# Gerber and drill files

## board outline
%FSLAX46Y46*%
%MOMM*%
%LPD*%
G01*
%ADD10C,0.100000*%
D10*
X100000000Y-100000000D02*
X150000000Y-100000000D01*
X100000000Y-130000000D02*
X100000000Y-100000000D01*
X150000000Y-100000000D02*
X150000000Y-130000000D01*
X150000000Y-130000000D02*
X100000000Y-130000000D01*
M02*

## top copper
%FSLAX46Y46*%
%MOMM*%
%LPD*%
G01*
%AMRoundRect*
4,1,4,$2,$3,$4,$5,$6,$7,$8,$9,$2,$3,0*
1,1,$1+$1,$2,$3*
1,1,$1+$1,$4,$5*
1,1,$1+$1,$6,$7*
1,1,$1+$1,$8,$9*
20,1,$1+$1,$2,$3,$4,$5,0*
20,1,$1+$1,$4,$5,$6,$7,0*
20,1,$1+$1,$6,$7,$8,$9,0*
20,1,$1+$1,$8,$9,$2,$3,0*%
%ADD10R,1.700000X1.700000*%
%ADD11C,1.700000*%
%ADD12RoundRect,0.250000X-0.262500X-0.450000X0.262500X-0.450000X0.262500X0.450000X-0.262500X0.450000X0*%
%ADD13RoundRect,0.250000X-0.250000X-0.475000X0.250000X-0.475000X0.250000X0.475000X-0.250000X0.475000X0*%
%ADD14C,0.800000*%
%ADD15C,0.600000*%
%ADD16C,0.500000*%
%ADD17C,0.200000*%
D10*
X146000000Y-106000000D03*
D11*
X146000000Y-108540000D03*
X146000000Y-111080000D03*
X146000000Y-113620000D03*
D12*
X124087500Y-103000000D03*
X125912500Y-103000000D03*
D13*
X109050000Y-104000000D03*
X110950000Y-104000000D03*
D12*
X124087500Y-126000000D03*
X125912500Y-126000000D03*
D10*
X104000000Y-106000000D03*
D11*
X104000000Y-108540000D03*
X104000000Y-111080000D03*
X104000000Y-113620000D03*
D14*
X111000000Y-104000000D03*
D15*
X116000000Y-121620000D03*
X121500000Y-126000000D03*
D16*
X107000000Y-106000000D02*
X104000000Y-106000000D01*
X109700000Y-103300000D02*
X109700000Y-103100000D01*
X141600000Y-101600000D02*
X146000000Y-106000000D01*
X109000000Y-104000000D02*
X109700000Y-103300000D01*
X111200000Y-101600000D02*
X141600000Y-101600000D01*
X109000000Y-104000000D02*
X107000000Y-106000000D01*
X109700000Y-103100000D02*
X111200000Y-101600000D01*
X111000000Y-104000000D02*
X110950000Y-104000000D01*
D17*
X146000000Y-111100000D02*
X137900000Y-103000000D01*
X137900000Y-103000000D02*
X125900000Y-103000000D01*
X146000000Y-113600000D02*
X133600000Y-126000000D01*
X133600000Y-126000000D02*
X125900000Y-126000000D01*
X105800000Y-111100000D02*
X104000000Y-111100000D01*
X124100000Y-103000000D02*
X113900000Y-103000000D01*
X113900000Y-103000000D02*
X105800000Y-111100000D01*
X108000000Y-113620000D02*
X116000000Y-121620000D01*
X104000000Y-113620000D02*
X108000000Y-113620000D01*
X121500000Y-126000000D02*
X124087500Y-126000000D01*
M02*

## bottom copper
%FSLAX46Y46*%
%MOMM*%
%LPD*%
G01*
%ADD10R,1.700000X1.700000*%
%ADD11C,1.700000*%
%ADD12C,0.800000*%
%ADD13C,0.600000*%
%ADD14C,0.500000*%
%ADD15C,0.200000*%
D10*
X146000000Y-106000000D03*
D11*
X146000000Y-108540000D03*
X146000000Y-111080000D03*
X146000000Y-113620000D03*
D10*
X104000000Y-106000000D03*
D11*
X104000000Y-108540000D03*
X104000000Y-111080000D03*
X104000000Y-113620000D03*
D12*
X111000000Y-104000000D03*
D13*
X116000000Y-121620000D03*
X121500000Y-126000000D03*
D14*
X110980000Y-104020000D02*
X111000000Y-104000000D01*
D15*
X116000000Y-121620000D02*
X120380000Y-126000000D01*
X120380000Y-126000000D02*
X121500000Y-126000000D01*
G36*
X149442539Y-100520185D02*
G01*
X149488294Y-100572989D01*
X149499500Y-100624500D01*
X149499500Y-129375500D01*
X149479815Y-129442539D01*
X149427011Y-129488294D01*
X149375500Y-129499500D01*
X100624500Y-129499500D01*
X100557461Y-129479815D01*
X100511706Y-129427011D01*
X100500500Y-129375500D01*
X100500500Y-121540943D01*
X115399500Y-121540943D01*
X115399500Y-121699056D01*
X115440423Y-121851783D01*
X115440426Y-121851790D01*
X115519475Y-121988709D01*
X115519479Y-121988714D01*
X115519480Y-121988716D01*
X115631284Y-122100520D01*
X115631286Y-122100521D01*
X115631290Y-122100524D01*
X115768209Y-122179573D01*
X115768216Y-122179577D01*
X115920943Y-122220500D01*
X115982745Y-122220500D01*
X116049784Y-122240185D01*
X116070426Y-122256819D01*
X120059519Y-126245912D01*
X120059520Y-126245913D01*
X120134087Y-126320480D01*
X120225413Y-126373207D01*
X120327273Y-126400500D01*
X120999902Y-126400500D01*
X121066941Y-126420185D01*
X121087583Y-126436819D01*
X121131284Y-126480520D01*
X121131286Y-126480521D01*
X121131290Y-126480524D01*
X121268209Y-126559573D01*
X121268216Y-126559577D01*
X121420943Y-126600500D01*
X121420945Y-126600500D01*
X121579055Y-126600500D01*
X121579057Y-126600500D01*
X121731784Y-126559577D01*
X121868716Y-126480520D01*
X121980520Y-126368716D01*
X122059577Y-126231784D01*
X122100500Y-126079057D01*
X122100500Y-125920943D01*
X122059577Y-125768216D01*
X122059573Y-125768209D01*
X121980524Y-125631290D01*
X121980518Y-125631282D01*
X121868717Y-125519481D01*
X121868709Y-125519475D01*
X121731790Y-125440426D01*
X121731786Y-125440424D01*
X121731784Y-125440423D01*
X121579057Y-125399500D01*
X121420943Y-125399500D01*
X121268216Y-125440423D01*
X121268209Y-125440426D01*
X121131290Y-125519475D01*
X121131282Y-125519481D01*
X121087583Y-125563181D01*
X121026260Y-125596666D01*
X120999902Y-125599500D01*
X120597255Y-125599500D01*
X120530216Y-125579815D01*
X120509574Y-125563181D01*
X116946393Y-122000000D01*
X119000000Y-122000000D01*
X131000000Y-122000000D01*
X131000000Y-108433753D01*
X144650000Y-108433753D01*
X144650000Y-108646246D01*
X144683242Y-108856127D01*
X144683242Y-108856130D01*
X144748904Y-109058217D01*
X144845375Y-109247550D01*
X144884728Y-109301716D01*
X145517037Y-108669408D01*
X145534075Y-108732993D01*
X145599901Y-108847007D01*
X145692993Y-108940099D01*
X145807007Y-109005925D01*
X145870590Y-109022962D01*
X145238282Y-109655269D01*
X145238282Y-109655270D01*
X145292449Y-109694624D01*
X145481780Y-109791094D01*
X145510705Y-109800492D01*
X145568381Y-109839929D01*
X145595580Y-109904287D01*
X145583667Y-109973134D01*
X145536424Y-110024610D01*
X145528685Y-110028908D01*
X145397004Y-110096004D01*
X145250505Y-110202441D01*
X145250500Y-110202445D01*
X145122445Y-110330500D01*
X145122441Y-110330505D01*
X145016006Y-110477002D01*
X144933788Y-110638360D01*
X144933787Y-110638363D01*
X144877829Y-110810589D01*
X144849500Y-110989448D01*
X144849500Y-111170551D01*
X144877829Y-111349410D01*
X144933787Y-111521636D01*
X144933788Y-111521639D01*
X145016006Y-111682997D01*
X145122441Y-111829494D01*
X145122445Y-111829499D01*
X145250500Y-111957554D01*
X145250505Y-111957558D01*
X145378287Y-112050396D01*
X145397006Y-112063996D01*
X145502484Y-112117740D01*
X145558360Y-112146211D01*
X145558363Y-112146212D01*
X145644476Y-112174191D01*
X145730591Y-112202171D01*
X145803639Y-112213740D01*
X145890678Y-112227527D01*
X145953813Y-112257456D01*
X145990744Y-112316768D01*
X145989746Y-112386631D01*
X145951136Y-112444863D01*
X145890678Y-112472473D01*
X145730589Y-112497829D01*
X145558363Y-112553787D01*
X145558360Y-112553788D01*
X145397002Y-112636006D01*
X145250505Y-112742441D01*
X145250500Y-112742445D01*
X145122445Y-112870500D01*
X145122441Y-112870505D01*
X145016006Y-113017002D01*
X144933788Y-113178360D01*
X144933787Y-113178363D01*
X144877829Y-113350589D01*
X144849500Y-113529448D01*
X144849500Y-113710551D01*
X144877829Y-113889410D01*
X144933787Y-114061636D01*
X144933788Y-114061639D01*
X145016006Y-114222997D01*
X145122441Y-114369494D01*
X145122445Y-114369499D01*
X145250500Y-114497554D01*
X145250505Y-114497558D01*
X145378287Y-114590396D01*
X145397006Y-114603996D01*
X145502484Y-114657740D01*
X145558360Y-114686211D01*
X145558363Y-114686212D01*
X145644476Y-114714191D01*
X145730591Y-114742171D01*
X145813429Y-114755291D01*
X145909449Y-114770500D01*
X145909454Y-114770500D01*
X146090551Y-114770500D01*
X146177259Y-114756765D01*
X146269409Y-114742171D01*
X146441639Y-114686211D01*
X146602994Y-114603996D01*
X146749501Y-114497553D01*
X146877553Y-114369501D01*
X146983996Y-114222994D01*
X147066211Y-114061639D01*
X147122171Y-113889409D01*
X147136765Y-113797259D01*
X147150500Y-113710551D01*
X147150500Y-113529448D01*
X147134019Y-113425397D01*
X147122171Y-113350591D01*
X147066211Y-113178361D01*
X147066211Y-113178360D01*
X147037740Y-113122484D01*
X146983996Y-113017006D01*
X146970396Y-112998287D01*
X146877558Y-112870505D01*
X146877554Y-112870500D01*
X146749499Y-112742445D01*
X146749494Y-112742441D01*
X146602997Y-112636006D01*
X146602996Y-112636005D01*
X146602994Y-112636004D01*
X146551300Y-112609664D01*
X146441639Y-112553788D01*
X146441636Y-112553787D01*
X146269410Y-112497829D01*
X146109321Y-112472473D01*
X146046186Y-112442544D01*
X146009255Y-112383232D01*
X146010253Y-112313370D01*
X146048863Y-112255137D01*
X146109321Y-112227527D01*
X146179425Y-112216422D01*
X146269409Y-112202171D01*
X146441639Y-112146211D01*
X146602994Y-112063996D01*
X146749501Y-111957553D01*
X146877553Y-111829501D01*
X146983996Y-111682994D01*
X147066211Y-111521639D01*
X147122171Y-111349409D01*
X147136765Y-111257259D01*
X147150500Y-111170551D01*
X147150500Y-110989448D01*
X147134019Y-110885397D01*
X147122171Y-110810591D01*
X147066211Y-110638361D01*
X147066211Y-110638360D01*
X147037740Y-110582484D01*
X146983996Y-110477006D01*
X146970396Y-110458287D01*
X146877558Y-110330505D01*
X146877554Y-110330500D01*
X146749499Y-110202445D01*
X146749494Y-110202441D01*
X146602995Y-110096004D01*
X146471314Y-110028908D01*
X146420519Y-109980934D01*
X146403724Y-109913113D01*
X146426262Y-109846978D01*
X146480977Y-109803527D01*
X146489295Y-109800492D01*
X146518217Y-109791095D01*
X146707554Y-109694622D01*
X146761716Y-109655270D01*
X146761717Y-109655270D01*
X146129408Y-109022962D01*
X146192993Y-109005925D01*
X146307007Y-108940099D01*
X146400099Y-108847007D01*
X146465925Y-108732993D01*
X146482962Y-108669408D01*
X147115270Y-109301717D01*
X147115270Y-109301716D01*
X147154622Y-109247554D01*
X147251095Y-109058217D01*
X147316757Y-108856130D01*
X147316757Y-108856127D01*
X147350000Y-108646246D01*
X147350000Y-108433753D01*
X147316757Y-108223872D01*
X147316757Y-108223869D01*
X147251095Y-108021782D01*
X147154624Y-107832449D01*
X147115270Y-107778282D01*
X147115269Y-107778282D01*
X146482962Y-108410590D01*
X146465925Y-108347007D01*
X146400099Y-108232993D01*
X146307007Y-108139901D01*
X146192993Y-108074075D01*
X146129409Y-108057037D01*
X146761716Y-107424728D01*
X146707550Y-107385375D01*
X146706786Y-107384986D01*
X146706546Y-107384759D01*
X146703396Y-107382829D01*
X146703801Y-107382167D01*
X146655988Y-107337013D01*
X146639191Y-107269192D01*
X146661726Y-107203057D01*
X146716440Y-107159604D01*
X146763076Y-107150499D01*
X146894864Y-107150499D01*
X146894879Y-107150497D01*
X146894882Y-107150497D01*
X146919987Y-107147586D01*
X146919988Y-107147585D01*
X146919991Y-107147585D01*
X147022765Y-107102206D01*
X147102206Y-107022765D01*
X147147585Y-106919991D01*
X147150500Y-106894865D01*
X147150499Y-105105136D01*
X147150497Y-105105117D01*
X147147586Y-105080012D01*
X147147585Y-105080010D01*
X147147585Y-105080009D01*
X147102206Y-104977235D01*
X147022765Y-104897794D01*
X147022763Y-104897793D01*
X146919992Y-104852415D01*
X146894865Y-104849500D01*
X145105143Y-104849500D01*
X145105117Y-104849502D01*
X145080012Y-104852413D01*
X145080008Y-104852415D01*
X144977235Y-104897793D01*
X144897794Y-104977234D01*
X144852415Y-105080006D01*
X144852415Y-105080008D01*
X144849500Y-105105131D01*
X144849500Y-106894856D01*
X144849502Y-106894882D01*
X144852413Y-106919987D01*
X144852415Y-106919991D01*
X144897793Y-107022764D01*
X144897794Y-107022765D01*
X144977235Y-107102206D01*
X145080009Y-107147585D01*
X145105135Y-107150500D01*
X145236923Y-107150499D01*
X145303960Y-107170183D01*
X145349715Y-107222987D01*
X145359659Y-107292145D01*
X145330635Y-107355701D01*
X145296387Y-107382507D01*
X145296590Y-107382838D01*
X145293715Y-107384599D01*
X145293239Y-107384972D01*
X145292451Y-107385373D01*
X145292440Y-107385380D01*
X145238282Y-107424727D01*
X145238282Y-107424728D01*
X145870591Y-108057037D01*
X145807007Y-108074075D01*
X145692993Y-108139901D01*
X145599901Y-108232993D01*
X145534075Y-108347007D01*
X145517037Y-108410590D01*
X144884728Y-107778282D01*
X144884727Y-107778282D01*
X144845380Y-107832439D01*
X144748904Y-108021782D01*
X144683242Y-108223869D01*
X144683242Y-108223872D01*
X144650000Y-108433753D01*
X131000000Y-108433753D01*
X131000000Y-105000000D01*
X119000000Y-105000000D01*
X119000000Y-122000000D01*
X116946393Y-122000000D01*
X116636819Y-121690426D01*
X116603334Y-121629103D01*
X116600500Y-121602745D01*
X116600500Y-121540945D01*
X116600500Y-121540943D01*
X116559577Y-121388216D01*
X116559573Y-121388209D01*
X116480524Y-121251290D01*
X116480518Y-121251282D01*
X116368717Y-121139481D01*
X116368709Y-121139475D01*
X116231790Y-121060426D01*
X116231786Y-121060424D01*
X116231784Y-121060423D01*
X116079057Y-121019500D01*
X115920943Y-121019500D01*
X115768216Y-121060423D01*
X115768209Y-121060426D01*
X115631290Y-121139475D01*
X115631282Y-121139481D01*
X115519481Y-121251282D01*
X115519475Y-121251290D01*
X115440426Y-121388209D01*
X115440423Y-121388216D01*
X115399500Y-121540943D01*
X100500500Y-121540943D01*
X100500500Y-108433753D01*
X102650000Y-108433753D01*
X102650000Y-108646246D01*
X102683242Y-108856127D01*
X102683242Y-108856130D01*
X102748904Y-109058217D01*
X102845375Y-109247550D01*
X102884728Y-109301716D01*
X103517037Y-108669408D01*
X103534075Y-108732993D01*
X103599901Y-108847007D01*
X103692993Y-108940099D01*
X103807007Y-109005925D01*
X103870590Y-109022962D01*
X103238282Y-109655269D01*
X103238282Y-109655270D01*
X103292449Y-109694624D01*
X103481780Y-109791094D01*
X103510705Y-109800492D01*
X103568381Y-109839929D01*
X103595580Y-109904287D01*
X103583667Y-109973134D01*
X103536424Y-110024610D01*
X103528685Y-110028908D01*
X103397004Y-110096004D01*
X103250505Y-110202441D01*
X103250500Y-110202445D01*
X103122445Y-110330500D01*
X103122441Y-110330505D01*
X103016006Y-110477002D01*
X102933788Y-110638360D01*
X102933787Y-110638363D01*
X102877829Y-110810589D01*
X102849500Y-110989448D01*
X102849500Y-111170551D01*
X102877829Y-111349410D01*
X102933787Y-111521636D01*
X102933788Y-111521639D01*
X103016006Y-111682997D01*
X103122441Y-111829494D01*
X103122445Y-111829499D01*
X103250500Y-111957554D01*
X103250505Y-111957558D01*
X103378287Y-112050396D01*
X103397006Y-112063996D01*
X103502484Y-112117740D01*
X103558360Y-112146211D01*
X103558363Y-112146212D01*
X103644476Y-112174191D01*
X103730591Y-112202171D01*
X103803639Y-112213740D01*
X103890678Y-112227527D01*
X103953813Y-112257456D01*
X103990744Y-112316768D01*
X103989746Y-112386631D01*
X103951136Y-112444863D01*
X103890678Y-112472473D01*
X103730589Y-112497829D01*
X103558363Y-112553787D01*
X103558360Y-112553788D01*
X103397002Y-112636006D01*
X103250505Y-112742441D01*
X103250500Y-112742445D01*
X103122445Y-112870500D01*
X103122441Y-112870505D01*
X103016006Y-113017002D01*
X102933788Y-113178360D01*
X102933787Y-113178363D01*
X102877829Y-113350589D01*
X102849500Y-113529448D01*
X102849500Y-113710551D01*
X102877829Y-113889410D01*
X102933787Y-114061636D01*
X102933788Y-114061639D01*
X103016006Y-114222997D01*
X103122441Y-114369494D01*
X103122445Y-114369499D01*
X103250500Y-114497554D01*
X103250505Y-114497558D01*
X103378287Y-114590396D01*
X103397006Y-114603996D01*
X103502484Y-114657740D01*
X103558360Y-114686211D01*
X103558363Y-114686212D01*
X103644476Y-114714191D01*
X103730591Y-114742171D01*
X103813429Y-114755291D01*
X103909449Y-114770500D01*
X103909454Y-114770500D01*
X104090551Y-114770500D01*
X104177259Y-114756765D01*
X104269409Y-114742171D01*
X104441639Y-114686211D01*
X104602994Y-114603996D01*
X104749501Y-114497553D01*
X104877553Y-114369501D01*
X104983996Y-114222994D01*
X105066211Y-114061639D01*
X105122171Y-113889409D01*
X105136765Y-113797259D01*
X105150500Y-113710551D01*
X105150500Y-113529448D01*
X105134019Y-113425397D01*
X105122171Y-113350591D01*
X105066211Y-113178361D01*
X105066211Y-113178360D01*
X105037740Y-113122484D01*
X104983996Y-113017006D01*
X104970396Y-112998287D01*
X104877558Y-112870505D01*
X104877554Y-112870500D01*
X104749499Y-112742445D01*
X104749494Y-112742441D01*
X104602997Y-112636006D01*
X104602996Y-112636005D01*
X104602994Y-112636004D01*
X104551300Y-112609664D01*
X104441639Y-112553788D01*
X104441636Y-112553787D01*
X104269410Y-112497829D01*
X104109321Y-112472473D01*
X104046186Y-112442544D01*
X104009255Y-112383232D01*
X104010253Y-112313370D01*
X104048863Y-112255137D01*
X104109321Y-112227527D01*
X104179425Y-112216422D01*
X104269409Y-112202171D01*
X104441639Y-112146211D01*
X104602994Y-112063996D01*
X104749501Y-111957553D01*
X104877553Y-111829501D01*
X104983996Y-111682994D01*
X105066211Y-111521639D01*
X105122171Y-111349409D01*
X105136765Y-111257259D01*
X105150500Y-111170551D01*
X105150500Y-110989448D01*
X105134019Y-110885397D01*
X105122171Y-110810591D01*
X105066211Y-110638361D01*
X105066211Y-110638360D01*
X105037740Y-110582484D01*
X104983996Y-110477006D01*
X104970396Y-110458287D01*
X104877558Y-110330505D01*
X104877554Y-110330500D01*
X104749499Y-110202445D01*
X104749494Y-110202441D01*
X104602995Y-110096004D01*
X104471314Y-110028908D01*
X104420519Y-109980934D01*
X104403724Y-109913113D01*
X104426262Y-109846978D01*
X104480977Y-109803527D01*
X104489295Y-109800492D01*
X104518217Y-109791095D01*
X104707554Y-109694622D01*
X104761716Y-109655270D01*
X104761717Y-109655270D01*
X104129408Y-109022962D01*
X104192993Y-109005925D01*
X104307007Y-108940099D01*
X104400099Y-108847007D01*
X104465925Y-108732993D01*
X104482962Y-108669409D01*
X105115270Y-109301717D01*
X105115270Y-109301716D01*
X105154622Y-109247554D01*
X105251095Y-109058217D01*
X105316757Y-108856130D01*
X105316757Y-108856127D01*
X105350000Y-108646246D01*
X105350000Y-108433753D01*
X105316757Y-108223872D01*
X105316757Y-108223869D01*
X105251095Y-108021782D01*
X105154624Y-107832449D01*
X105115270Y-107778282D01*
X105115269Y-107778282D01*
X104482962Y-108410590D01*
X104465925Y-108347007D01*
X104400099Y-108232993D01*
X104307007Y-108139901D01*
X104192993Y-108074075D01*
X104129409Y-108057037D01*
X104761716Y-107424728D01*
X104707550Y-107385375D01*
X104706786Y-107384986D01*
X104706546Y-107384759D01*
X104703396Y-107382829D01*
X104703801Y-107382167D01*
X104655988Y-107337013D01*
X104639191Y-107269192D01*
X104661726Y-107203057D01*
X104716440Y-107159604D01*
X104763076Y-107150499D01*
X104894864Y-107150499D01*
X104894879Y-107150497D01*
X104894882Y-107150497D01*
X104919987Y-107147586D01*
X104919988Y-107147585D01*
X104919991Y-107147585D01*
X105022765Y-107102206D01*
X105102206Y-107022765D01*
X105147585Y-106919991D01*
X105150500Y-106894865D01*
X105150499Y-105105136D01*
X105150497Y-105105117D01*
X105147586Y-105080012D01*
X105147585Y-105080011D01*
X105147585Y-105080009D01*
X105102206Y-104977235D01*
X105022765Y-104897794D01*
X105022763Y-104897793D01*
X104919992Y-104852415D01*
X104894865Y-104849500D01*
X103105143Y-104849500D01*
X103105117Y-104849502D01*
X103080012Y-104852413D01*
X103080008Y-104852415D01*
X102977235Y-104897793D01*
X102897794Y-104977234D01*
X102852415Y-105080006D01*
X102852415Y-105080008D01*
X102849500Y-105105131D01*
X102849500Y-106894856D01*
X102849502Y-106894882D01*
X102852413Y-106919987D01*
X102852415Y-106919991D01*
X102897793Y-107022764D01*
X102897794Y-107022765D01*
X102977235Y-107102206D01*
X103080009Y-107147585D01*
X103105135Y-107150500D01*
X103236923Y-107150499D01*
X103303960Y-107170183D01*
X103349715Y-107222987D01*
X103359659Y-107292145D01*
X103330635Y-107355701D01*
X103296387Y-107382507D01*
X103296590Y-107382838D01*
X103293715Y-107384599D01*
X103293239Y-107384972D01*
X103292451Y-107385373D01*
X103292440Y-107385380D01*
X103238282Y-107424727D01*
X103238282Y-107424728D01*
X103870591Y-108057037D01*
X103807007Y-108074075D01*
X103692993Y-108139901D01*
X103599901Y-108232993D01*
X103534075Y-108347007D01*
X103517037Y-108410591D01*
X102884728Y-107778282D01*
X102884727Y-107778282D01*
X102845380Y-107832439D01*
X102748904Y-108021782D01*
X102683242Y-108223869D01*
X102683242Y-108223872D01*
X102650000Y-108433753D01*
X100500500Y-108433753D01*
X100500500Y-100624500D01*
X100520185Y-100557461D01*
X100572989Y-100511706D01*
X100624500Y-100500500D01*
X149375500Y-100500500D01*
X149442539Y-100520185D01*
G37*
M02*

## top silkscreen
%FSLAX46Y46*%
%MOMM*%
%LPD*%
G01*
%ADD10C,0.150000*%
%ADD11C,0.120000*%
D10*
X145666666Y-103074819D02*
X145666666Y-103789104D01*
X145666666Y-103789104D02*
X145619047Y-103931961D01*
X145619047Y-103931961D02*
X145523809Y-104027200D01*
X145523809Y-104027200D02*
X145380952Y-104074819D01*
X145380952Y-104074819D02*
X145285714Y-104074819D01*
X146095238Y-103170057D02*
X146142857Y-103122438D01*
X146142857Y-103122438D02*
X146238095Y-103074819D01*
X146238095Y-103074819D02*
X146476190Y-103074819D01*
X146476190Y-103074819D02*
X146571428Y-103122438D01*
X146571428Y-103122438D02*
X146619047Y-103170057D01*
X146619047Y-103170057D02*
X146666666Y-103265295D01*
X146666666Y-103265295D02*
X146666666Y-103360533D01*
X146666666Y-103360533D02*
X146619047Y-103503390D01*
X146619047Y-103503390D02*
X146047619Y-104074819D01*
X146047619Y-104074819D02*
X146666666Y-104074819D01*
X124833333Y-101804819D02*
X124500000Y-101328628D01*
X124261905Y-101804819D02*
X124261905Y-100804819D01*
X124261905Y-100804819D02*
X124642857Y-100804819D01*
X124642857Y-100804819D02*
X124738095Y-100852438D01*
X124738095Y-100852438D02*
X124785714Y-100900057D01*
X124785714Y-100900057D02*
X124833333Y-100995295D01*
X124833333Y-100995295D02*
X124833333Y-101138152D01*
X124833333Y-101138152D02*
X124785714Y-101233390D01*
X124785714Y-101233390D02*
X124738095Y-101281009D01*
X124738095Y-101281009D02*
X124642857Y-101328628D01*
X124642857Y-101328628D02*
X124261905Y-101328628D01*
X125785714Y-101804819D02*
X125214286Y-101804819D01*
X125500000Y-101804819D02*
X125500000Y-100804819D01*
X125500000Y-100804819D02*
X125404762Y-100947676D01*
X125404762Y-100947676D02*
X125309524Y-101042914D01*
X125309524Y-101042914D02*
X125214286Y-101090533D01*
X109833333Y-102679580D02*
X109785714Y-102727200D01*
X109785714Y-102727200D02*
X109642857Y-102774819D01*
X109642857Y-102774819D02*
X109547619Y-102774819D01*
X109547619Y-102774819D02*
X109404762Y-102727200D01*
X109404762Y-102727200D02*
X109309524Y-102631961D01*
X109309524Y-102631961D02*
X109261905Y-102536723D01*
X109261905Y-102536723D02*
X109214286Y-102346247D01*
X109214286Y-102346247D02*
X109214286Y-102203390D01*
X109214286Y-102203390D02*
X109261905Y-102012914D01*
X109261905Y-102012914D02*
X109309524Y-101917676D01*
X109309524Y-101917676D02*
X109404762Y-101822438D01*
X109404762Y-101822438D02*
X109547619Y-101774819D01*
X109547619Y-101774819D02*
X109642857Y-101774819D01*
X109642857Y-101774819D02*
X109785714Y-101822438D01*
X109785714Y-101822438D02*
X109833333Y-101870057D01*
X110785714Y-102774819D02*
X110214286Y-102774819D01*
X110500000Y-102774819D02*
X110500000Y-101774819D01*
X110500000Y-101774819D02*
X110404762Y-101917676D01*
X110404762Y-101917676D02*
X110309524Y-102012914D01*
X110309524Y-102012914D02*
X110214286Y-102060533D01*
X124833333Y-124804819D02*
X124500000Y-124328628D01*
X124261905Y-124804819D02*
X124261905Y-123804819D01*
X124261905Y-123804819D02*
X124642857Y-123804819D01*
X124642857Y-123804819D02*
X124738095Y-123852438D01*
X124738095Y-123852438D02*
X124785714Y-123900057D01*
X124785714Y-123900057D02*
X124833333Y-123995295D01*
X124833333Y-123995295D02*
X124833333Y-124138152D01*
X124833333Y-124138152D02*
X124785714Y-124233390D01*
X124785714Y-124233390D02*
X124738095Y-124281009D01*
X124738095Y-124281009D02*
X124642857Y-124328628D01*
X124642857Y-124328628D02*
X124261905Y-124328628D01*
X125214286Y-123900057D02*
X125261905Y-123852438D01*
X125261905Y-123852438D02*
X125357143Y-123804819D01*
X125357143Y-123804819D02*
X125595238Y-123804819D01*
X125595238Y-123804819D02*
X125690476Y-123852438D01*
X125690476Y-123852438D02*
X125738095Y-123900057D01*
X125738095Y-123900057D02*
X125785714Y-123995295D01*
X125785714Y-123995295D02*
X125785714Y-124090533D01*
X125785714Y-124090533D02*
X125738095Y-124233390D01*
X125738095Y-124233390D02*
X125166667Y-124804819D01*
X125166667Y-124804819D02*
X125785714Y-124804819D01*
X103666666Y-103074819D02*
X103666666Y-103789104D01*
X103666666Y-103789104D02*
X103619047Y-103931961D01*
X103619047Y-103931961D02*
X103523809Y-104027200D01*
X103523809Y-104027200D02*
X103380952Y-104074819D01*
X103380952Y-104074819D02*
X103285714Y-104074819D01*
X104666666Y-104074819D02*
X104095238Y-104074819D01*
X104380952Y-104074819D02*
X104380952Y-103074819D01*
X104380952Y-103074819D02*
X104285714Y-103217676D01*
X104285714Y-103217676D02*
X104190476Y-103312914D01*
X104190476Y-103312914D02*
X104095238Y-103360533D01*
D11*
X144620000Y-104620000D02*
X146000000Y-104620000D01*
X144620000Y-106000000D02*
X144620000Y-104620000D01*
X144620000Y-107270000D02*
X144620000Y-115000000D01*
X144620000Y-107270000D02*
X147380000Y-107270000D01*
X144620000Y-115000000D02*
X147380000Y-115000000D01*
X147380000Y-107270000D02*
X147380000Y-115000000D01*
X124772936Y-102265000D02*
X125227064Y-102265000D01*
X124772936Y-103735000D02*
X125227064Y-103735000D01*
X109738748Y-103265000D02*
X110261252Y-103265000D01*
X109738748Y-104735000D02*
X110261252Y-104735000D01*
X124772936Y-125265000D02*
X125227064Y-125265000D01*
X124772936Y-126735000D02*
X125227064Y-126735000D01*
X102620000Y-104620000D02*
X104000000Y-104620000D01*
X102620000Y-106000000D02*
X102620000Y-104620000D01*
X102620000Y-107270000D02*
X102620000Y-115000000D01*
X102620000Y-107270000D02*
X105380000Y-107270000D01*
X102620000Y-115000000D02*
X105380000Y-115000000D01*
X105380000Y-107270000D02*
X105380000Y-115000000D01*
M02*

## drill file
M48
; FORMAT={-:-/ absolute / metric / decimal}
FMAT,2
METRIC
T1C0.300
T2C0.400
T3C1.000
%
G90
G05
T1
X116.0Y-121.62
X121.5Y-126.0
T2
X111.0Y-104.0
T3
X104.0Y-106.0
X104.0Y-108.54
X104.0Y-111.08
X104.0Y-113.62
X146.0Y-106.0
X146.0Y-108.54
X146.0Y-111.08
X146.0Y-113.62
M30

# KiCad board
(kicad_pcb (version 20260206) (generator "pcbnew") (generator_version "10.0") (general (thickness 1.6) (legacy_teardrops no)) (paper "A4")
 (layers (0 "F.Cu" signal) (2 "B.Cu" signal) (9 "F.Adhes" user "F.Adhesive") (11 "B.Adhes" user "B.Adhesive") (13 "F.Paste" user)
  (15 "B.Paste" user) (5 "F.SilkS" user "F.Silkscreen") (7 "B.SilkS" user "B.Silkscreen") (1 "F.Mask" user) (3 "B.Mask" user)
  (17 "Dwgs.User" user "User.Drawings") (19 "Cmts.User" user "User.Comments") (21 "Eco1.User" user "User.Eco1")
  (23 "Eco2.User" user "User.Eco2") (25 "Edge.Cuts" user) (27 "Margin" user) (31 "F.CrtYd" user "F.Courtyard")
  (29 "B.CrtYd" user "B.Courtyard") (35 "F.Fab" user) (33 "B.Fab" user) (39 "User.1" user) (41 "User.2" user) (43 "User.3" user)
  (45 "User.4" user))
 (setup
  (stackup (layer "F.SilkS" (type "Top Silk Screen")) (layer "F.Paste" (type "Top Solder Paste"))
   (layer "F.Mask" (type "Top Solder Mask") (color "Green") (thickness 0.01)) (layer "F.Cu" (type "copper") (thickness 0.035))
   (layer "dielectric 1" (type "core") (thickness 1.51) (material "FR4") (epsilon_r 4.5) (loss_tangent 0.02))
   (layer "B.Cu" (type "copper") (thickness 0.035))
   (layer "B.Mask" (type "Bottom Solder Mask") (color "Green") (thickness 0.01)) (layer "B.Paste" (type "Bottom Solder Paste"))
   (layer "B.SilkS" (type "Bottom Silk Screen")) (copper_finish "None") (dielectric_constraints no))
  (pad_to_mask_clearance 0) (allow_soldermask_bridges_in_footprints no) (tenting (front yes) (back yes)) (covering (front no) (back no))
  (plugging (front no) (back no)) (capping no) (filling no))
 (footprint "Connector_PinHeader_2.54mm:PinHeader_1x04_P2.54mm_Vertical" (layer "F.Cu") (at 146 106)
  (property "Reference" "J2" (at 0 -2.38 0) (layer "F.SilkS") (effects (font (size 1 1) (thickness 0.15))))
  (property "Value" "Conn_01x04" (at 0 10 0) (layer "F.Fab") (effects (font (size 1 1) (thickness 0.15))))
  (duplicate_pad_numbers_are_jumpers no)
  (fp_line (start -1.38 -1.38) (end 0 -1.38) (stroke (width 0.12) (type solid)) (layer "F.SilkS"))
  (fp_line (start -1.38 0) (end -1.38 -1.38) (stroke (width 0.12) (type solid)) (layer "F.SilkS"))
  (fp_line (start -1.38 1.27) (end -1.38 9) (stroke (width 0.12) (type solid)) (layer "F.SilkS"))
  (fp_line (start -1.38 1.27) (end 1.38 1.27) (stroke (width 0.12) (type solid)) (layer "F.SilkS"))
  (fp_line (start -1.38 9) (end 1.38 9) (stroke (width 0.12) (type solid)) (layer "F.SilkS"))
  (fp_line (start 1.38 1.27) (end 1.38 9) (stroke (width 0.12) (type solid)) (layer "F.SilkS"))
  (pad "1" thru_hole rect (at 0 0) (size 1.7 1.7) (drill 1) (layers "*.Cu" "*.Mask") (remove_unused_layers no) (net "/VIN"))
  (pad "2" thru_hole circle (at 0 2.54) (size 1.7 1.7) (drill 1) (layers "*.Cu" "*.Mask") (remove_unused_layers no) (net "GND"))
  (pad "3" thru_hole circle (at 0 5.08) (size 1.7 1.7) (drill 1) (layers "*.Cu" "*.Mask") (remove_unused_layers no) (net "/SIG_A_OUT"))
  (pad "4" thru_hole circle (at 0 7.62) (size 1.7 1.7) (drill 1) (layers "*.Cu" "*.Mask") (remove_unused_layers no) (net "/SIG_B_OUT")))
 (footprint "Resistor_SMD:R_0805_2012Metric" (layer "F.Cu") (at 125 103)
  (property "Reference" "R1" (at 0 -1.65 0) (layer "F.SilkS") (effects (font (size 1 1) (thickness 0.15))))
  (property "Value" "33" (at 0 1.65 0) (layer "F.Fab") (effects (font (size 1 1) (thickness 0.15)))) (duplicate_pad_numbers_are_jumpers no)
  (fp_line (start -0.227064 -0.735) (end 0.227064 -0.735) (stroke (width 0.12) (type solid)) (layer "F.SilkS"))
  (fp_line (start -0.227064 0.735) (end 0.227064 0.735) (stroke (width 0.12) (type solid)) (layer "F.SilkS"))
  (pad "1" smd roundrect (at -0.9125 0) (size 1.025 1.4) (layers "F.Cu" "F.Mask" "F.Paste") (roundrect_rratio 0.243902) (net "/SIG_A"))
  (pad "2" smd roundrect (at 0.9125 0) (size 1.025 1.4) (layers "F.Cu" "F.Mask" "F.Paste") (roundrect_rratio 0.243902) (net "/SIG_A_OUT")))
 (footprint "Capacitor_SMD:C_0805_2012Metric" (layer "F.Cu") (at 110 104)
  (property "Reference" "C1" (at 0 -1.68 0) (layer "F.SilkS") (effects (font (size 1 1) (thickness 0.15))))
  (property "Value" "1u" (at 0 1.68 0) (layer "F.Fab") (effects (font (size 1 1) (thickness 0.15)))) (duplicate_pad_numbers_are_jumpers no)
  (fp_line (start -0.261252 -0.735) (end 0.261252 -0.735) (stroke (width 0.12) (type solid)) (layer "F.SilkS"))
  (fp_line (start -0.261252 0.735) (end 0.261252 0.735) (stroke (width 0.12) (type solid)) (layer "F.SilkS"))
  (pad "1" smd roundrect (at -0.95 0) (size 1 1.45) (layers "F.Cu" "F.Mask" "F.Paste") (roundrect_rratio 0.25) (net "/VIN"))
  (pad "2" smd roundrect (at 0.95 0) (size 1 1.45) (layers "F.Cu" "F.Mask" "F.Paste") (roundrect_rratio 0.25) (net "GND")))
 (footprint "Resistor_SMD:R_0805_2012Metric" (layer "F.Cu") (at 125 126)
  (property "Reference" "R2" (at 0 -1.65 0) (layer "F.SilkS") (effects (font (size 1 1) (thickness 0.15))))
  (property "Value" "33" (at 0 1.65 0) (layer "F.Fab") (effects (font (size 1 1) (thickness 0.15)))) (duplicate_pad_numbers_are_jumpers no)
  (fp_line (start -0.227064 -0.735) (end 0.227064 -0.735) (stroke (width 0.12) (type solid)) (layer "F.SilkS"))
  (fp_line (start -0.227064 0.735) (end 0.227064 0.735) (stroke (width 0.12) (type solid)) (layer "F.SilkS"))
  (pad "1" smd roundrect (at -0.9125 0) (size 1.025 1.4) (layers "F.Cu" "F.Mask" "F.Paste") (roundrect_rratio 0.243902) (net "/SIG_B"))
  (pad "2" smd roundrect (at 0.9125 0) (size 1.025 1.4) (layers "F.Cu" "F.Mask" "F.Paste") (roundrect_rratio 0.243902) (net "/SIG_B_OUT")))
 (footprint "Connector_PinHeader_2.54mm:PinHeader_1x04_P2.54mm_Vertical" (layer "F.Cu") (at 104 106)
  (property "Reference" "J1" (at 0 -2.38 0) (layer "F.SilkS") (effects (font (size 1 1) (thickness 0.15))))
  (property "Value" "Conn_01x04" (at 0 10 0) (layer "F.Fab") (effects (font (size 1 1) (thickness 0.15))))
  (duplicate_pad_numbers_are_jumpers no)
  (fp_line (start -1.38 -1.38) (end 0 -1.38) (stroke (width 0.12) (type solid)) (layer "F.SilkS"))
  (fp_line (start -1.38 0) (end -1.38 -1.38) (stroke (width 0.12) (type solid)) (layer "F.SilkS"))
  (fp_line (start -1.38 1.27) (end -1.38 9) (stroke (width 0.12) (type solid)) (layer "F.SilkS"))
  (fp_line (start -1.38 1.27) (end 1.38 1.27) (stroke (width 0.12) (type solid)) (layer "F.SilkS"))
  (fp_line (start -1.38 9) (end 1.38 9) (stroke (width 0.12) (type solid)) (layer "F.SilkS"))
  (fp_line (start 1.38 1.27) (end 1.38 9) (stroke (width 0.12) (type solid)) (layer "F.SilkS"))
  (pad "1" thru_hole rect (at 0 0) (size 1.7 1.7) (drill 1) (layers "*.Cu" "*.Mask") (remove_unused_layers no) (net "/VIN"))
  (pad "2" thru_hole circle (at 0 2.54) (size 1.7 1.7) (drill 1) (layers "*.Cu" "*.Mask") (remove_unused_layers no) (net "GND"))
  (pad "3" thru_hole circle (at 0 5.08) (size 1.7 1.7) (drill 1) (layers "*.Cu" "*.Mask") (remove_unused_layers no) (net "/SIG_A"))
  (pad "4" thru_hole circle (at 0 7.62) (size 1.7 1.7) (drill 1) (layers "*.Cu" "*.Mask") (remove_unused_layers no) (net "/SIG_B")))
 (gr_line (start 100 100) (end 150 100) (stroke (width 0.1) (type default)) (layer "Edge.Cuts"))
 (gr_line (start 100 130) (end 100 100) (stroke (width 0.1) (type default)) (layer "Edge.Cuts"))
 (gr_line (start 150 100) (end 150 130) (stroke (width 0.1) (type default)) (layer "Edge.Cuts"))
 (gr_line (start 150 130) (end 100 130) (stroke (width 0.1) (type default)) (layer "Edge.Cuts"))
 (segment (start 107 106) (end 104 106) (width 0.5) (layer "F.Cu") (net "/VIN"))
 (segment (start 109.7 103.3) (end 109.7 103.1) (width 0.5) (layer "F.Cu") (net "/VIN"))
 (segment (start 141.6 101.6) (end 146 106) (width 0.5) (layer "F.Cu") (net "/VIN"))
 (segment (start 109 104) (end 109.7 103.3) (width 0.5) (layer "F.Cu") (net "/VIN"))
 (segment (start 111.2 101.6) (end 141.6 101.6) (width 0.5) (layer "F.Cu") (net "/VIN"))
 (segment (start 109 104) (end 107 106) (width 0.5) (layer "F.Cu") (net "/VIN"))
 (segment (start 109.7 103.1) (end 111.2 101.6) (width 0.5) (layer "F.Cu") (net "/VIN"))
 (segment (start 111 104) (end 110.95 104) (width 0.5) (layer "F.Cu") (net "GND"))
 (via (at 111 104) (size 0.8) (drill 0.4) (layers "F.Cu" "B.Cu") (capping yes) (filling yes) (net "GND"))
 (segment (start 110.98 104.02) (end 111 104) (width 0.5) (layer "B.Cu") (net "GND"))
 (segment (start 146 111.1) (end 137.9 103) (width 0.2) (layer "F.Cu") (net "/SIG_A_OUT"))
 (segment (start 137.9 103) (end 125.9 103) (width 0.2) (layer "F.Cu") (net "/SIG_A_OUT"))
 (segment (start 146 113.6) (end 133.6 126) (width 0.2) (layer "F.Cu") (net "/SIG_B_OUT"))
 (segment (start 133.6 126) (end 125.9 126) (width 0.2) (layer "F.Cu") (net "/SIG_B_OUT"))
 (segment (start 105.8 111.1) (end 104 111.1) (width 0.2) (layer "F.Cu") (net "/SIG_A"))
 (segment (start 124.1 103) (end 113.9 103) (width 0.2) (layer "F.Cu") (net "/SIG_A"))
 (segment (start 113.9 103) (end 105.8 111.1) (width 0.2) (layer "F.Cu") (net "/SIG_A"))
 (segment (start 108 113.62) (end 116 121.62) (width 0.2) (locked yes) (layer "F.Cu") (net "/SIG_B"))
 (segment (start 104 113.62) (end 108 113.62) (width 0.2) (locked yes) (layer "F.Cu") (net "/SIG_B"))
 (segment (start 121.5 126) (end 124.0875 126) (width 0.2) (locked yes) (layer "F.Cu") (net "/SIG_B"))
 (via (at 116 121.62) (size 0.6) (drill 0.3) (layers "F.Cu" "B.Cu") (locked yes) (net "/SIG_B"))
 (via (at 121.5 126) (size 0.6) (drill 0.3) (layers "F.Cu" "B.Cu") (locked yes) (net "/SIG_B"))
 (segment (start 116 121.62) (end 120.38 126) (width 0.2) (locked yes) (layer "B.Cu") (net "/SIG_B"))
 (segment (start 120.38 126) (end 121.5 126) (width 0.2) (locked yes) (layer "B.Cu") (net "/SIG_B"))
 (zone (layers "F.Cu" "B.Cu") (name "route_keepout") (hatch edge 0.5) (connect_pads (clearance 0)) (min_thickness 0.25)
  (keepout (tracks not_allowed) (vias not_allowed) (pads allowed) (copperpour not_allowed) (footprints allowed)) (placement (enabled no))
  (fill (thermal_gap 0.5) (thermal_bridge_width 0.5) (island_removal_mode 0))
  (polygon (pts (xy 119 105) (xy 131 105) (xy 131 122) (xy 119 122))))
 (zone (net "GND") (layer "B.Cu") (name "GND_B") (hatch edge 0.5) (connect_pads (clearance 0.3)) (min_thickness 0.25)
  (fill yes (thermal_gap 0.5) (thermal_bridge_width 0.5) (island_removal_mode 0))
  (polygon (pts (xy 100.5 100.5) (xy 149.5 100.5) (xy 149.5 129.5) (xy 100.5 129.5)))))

